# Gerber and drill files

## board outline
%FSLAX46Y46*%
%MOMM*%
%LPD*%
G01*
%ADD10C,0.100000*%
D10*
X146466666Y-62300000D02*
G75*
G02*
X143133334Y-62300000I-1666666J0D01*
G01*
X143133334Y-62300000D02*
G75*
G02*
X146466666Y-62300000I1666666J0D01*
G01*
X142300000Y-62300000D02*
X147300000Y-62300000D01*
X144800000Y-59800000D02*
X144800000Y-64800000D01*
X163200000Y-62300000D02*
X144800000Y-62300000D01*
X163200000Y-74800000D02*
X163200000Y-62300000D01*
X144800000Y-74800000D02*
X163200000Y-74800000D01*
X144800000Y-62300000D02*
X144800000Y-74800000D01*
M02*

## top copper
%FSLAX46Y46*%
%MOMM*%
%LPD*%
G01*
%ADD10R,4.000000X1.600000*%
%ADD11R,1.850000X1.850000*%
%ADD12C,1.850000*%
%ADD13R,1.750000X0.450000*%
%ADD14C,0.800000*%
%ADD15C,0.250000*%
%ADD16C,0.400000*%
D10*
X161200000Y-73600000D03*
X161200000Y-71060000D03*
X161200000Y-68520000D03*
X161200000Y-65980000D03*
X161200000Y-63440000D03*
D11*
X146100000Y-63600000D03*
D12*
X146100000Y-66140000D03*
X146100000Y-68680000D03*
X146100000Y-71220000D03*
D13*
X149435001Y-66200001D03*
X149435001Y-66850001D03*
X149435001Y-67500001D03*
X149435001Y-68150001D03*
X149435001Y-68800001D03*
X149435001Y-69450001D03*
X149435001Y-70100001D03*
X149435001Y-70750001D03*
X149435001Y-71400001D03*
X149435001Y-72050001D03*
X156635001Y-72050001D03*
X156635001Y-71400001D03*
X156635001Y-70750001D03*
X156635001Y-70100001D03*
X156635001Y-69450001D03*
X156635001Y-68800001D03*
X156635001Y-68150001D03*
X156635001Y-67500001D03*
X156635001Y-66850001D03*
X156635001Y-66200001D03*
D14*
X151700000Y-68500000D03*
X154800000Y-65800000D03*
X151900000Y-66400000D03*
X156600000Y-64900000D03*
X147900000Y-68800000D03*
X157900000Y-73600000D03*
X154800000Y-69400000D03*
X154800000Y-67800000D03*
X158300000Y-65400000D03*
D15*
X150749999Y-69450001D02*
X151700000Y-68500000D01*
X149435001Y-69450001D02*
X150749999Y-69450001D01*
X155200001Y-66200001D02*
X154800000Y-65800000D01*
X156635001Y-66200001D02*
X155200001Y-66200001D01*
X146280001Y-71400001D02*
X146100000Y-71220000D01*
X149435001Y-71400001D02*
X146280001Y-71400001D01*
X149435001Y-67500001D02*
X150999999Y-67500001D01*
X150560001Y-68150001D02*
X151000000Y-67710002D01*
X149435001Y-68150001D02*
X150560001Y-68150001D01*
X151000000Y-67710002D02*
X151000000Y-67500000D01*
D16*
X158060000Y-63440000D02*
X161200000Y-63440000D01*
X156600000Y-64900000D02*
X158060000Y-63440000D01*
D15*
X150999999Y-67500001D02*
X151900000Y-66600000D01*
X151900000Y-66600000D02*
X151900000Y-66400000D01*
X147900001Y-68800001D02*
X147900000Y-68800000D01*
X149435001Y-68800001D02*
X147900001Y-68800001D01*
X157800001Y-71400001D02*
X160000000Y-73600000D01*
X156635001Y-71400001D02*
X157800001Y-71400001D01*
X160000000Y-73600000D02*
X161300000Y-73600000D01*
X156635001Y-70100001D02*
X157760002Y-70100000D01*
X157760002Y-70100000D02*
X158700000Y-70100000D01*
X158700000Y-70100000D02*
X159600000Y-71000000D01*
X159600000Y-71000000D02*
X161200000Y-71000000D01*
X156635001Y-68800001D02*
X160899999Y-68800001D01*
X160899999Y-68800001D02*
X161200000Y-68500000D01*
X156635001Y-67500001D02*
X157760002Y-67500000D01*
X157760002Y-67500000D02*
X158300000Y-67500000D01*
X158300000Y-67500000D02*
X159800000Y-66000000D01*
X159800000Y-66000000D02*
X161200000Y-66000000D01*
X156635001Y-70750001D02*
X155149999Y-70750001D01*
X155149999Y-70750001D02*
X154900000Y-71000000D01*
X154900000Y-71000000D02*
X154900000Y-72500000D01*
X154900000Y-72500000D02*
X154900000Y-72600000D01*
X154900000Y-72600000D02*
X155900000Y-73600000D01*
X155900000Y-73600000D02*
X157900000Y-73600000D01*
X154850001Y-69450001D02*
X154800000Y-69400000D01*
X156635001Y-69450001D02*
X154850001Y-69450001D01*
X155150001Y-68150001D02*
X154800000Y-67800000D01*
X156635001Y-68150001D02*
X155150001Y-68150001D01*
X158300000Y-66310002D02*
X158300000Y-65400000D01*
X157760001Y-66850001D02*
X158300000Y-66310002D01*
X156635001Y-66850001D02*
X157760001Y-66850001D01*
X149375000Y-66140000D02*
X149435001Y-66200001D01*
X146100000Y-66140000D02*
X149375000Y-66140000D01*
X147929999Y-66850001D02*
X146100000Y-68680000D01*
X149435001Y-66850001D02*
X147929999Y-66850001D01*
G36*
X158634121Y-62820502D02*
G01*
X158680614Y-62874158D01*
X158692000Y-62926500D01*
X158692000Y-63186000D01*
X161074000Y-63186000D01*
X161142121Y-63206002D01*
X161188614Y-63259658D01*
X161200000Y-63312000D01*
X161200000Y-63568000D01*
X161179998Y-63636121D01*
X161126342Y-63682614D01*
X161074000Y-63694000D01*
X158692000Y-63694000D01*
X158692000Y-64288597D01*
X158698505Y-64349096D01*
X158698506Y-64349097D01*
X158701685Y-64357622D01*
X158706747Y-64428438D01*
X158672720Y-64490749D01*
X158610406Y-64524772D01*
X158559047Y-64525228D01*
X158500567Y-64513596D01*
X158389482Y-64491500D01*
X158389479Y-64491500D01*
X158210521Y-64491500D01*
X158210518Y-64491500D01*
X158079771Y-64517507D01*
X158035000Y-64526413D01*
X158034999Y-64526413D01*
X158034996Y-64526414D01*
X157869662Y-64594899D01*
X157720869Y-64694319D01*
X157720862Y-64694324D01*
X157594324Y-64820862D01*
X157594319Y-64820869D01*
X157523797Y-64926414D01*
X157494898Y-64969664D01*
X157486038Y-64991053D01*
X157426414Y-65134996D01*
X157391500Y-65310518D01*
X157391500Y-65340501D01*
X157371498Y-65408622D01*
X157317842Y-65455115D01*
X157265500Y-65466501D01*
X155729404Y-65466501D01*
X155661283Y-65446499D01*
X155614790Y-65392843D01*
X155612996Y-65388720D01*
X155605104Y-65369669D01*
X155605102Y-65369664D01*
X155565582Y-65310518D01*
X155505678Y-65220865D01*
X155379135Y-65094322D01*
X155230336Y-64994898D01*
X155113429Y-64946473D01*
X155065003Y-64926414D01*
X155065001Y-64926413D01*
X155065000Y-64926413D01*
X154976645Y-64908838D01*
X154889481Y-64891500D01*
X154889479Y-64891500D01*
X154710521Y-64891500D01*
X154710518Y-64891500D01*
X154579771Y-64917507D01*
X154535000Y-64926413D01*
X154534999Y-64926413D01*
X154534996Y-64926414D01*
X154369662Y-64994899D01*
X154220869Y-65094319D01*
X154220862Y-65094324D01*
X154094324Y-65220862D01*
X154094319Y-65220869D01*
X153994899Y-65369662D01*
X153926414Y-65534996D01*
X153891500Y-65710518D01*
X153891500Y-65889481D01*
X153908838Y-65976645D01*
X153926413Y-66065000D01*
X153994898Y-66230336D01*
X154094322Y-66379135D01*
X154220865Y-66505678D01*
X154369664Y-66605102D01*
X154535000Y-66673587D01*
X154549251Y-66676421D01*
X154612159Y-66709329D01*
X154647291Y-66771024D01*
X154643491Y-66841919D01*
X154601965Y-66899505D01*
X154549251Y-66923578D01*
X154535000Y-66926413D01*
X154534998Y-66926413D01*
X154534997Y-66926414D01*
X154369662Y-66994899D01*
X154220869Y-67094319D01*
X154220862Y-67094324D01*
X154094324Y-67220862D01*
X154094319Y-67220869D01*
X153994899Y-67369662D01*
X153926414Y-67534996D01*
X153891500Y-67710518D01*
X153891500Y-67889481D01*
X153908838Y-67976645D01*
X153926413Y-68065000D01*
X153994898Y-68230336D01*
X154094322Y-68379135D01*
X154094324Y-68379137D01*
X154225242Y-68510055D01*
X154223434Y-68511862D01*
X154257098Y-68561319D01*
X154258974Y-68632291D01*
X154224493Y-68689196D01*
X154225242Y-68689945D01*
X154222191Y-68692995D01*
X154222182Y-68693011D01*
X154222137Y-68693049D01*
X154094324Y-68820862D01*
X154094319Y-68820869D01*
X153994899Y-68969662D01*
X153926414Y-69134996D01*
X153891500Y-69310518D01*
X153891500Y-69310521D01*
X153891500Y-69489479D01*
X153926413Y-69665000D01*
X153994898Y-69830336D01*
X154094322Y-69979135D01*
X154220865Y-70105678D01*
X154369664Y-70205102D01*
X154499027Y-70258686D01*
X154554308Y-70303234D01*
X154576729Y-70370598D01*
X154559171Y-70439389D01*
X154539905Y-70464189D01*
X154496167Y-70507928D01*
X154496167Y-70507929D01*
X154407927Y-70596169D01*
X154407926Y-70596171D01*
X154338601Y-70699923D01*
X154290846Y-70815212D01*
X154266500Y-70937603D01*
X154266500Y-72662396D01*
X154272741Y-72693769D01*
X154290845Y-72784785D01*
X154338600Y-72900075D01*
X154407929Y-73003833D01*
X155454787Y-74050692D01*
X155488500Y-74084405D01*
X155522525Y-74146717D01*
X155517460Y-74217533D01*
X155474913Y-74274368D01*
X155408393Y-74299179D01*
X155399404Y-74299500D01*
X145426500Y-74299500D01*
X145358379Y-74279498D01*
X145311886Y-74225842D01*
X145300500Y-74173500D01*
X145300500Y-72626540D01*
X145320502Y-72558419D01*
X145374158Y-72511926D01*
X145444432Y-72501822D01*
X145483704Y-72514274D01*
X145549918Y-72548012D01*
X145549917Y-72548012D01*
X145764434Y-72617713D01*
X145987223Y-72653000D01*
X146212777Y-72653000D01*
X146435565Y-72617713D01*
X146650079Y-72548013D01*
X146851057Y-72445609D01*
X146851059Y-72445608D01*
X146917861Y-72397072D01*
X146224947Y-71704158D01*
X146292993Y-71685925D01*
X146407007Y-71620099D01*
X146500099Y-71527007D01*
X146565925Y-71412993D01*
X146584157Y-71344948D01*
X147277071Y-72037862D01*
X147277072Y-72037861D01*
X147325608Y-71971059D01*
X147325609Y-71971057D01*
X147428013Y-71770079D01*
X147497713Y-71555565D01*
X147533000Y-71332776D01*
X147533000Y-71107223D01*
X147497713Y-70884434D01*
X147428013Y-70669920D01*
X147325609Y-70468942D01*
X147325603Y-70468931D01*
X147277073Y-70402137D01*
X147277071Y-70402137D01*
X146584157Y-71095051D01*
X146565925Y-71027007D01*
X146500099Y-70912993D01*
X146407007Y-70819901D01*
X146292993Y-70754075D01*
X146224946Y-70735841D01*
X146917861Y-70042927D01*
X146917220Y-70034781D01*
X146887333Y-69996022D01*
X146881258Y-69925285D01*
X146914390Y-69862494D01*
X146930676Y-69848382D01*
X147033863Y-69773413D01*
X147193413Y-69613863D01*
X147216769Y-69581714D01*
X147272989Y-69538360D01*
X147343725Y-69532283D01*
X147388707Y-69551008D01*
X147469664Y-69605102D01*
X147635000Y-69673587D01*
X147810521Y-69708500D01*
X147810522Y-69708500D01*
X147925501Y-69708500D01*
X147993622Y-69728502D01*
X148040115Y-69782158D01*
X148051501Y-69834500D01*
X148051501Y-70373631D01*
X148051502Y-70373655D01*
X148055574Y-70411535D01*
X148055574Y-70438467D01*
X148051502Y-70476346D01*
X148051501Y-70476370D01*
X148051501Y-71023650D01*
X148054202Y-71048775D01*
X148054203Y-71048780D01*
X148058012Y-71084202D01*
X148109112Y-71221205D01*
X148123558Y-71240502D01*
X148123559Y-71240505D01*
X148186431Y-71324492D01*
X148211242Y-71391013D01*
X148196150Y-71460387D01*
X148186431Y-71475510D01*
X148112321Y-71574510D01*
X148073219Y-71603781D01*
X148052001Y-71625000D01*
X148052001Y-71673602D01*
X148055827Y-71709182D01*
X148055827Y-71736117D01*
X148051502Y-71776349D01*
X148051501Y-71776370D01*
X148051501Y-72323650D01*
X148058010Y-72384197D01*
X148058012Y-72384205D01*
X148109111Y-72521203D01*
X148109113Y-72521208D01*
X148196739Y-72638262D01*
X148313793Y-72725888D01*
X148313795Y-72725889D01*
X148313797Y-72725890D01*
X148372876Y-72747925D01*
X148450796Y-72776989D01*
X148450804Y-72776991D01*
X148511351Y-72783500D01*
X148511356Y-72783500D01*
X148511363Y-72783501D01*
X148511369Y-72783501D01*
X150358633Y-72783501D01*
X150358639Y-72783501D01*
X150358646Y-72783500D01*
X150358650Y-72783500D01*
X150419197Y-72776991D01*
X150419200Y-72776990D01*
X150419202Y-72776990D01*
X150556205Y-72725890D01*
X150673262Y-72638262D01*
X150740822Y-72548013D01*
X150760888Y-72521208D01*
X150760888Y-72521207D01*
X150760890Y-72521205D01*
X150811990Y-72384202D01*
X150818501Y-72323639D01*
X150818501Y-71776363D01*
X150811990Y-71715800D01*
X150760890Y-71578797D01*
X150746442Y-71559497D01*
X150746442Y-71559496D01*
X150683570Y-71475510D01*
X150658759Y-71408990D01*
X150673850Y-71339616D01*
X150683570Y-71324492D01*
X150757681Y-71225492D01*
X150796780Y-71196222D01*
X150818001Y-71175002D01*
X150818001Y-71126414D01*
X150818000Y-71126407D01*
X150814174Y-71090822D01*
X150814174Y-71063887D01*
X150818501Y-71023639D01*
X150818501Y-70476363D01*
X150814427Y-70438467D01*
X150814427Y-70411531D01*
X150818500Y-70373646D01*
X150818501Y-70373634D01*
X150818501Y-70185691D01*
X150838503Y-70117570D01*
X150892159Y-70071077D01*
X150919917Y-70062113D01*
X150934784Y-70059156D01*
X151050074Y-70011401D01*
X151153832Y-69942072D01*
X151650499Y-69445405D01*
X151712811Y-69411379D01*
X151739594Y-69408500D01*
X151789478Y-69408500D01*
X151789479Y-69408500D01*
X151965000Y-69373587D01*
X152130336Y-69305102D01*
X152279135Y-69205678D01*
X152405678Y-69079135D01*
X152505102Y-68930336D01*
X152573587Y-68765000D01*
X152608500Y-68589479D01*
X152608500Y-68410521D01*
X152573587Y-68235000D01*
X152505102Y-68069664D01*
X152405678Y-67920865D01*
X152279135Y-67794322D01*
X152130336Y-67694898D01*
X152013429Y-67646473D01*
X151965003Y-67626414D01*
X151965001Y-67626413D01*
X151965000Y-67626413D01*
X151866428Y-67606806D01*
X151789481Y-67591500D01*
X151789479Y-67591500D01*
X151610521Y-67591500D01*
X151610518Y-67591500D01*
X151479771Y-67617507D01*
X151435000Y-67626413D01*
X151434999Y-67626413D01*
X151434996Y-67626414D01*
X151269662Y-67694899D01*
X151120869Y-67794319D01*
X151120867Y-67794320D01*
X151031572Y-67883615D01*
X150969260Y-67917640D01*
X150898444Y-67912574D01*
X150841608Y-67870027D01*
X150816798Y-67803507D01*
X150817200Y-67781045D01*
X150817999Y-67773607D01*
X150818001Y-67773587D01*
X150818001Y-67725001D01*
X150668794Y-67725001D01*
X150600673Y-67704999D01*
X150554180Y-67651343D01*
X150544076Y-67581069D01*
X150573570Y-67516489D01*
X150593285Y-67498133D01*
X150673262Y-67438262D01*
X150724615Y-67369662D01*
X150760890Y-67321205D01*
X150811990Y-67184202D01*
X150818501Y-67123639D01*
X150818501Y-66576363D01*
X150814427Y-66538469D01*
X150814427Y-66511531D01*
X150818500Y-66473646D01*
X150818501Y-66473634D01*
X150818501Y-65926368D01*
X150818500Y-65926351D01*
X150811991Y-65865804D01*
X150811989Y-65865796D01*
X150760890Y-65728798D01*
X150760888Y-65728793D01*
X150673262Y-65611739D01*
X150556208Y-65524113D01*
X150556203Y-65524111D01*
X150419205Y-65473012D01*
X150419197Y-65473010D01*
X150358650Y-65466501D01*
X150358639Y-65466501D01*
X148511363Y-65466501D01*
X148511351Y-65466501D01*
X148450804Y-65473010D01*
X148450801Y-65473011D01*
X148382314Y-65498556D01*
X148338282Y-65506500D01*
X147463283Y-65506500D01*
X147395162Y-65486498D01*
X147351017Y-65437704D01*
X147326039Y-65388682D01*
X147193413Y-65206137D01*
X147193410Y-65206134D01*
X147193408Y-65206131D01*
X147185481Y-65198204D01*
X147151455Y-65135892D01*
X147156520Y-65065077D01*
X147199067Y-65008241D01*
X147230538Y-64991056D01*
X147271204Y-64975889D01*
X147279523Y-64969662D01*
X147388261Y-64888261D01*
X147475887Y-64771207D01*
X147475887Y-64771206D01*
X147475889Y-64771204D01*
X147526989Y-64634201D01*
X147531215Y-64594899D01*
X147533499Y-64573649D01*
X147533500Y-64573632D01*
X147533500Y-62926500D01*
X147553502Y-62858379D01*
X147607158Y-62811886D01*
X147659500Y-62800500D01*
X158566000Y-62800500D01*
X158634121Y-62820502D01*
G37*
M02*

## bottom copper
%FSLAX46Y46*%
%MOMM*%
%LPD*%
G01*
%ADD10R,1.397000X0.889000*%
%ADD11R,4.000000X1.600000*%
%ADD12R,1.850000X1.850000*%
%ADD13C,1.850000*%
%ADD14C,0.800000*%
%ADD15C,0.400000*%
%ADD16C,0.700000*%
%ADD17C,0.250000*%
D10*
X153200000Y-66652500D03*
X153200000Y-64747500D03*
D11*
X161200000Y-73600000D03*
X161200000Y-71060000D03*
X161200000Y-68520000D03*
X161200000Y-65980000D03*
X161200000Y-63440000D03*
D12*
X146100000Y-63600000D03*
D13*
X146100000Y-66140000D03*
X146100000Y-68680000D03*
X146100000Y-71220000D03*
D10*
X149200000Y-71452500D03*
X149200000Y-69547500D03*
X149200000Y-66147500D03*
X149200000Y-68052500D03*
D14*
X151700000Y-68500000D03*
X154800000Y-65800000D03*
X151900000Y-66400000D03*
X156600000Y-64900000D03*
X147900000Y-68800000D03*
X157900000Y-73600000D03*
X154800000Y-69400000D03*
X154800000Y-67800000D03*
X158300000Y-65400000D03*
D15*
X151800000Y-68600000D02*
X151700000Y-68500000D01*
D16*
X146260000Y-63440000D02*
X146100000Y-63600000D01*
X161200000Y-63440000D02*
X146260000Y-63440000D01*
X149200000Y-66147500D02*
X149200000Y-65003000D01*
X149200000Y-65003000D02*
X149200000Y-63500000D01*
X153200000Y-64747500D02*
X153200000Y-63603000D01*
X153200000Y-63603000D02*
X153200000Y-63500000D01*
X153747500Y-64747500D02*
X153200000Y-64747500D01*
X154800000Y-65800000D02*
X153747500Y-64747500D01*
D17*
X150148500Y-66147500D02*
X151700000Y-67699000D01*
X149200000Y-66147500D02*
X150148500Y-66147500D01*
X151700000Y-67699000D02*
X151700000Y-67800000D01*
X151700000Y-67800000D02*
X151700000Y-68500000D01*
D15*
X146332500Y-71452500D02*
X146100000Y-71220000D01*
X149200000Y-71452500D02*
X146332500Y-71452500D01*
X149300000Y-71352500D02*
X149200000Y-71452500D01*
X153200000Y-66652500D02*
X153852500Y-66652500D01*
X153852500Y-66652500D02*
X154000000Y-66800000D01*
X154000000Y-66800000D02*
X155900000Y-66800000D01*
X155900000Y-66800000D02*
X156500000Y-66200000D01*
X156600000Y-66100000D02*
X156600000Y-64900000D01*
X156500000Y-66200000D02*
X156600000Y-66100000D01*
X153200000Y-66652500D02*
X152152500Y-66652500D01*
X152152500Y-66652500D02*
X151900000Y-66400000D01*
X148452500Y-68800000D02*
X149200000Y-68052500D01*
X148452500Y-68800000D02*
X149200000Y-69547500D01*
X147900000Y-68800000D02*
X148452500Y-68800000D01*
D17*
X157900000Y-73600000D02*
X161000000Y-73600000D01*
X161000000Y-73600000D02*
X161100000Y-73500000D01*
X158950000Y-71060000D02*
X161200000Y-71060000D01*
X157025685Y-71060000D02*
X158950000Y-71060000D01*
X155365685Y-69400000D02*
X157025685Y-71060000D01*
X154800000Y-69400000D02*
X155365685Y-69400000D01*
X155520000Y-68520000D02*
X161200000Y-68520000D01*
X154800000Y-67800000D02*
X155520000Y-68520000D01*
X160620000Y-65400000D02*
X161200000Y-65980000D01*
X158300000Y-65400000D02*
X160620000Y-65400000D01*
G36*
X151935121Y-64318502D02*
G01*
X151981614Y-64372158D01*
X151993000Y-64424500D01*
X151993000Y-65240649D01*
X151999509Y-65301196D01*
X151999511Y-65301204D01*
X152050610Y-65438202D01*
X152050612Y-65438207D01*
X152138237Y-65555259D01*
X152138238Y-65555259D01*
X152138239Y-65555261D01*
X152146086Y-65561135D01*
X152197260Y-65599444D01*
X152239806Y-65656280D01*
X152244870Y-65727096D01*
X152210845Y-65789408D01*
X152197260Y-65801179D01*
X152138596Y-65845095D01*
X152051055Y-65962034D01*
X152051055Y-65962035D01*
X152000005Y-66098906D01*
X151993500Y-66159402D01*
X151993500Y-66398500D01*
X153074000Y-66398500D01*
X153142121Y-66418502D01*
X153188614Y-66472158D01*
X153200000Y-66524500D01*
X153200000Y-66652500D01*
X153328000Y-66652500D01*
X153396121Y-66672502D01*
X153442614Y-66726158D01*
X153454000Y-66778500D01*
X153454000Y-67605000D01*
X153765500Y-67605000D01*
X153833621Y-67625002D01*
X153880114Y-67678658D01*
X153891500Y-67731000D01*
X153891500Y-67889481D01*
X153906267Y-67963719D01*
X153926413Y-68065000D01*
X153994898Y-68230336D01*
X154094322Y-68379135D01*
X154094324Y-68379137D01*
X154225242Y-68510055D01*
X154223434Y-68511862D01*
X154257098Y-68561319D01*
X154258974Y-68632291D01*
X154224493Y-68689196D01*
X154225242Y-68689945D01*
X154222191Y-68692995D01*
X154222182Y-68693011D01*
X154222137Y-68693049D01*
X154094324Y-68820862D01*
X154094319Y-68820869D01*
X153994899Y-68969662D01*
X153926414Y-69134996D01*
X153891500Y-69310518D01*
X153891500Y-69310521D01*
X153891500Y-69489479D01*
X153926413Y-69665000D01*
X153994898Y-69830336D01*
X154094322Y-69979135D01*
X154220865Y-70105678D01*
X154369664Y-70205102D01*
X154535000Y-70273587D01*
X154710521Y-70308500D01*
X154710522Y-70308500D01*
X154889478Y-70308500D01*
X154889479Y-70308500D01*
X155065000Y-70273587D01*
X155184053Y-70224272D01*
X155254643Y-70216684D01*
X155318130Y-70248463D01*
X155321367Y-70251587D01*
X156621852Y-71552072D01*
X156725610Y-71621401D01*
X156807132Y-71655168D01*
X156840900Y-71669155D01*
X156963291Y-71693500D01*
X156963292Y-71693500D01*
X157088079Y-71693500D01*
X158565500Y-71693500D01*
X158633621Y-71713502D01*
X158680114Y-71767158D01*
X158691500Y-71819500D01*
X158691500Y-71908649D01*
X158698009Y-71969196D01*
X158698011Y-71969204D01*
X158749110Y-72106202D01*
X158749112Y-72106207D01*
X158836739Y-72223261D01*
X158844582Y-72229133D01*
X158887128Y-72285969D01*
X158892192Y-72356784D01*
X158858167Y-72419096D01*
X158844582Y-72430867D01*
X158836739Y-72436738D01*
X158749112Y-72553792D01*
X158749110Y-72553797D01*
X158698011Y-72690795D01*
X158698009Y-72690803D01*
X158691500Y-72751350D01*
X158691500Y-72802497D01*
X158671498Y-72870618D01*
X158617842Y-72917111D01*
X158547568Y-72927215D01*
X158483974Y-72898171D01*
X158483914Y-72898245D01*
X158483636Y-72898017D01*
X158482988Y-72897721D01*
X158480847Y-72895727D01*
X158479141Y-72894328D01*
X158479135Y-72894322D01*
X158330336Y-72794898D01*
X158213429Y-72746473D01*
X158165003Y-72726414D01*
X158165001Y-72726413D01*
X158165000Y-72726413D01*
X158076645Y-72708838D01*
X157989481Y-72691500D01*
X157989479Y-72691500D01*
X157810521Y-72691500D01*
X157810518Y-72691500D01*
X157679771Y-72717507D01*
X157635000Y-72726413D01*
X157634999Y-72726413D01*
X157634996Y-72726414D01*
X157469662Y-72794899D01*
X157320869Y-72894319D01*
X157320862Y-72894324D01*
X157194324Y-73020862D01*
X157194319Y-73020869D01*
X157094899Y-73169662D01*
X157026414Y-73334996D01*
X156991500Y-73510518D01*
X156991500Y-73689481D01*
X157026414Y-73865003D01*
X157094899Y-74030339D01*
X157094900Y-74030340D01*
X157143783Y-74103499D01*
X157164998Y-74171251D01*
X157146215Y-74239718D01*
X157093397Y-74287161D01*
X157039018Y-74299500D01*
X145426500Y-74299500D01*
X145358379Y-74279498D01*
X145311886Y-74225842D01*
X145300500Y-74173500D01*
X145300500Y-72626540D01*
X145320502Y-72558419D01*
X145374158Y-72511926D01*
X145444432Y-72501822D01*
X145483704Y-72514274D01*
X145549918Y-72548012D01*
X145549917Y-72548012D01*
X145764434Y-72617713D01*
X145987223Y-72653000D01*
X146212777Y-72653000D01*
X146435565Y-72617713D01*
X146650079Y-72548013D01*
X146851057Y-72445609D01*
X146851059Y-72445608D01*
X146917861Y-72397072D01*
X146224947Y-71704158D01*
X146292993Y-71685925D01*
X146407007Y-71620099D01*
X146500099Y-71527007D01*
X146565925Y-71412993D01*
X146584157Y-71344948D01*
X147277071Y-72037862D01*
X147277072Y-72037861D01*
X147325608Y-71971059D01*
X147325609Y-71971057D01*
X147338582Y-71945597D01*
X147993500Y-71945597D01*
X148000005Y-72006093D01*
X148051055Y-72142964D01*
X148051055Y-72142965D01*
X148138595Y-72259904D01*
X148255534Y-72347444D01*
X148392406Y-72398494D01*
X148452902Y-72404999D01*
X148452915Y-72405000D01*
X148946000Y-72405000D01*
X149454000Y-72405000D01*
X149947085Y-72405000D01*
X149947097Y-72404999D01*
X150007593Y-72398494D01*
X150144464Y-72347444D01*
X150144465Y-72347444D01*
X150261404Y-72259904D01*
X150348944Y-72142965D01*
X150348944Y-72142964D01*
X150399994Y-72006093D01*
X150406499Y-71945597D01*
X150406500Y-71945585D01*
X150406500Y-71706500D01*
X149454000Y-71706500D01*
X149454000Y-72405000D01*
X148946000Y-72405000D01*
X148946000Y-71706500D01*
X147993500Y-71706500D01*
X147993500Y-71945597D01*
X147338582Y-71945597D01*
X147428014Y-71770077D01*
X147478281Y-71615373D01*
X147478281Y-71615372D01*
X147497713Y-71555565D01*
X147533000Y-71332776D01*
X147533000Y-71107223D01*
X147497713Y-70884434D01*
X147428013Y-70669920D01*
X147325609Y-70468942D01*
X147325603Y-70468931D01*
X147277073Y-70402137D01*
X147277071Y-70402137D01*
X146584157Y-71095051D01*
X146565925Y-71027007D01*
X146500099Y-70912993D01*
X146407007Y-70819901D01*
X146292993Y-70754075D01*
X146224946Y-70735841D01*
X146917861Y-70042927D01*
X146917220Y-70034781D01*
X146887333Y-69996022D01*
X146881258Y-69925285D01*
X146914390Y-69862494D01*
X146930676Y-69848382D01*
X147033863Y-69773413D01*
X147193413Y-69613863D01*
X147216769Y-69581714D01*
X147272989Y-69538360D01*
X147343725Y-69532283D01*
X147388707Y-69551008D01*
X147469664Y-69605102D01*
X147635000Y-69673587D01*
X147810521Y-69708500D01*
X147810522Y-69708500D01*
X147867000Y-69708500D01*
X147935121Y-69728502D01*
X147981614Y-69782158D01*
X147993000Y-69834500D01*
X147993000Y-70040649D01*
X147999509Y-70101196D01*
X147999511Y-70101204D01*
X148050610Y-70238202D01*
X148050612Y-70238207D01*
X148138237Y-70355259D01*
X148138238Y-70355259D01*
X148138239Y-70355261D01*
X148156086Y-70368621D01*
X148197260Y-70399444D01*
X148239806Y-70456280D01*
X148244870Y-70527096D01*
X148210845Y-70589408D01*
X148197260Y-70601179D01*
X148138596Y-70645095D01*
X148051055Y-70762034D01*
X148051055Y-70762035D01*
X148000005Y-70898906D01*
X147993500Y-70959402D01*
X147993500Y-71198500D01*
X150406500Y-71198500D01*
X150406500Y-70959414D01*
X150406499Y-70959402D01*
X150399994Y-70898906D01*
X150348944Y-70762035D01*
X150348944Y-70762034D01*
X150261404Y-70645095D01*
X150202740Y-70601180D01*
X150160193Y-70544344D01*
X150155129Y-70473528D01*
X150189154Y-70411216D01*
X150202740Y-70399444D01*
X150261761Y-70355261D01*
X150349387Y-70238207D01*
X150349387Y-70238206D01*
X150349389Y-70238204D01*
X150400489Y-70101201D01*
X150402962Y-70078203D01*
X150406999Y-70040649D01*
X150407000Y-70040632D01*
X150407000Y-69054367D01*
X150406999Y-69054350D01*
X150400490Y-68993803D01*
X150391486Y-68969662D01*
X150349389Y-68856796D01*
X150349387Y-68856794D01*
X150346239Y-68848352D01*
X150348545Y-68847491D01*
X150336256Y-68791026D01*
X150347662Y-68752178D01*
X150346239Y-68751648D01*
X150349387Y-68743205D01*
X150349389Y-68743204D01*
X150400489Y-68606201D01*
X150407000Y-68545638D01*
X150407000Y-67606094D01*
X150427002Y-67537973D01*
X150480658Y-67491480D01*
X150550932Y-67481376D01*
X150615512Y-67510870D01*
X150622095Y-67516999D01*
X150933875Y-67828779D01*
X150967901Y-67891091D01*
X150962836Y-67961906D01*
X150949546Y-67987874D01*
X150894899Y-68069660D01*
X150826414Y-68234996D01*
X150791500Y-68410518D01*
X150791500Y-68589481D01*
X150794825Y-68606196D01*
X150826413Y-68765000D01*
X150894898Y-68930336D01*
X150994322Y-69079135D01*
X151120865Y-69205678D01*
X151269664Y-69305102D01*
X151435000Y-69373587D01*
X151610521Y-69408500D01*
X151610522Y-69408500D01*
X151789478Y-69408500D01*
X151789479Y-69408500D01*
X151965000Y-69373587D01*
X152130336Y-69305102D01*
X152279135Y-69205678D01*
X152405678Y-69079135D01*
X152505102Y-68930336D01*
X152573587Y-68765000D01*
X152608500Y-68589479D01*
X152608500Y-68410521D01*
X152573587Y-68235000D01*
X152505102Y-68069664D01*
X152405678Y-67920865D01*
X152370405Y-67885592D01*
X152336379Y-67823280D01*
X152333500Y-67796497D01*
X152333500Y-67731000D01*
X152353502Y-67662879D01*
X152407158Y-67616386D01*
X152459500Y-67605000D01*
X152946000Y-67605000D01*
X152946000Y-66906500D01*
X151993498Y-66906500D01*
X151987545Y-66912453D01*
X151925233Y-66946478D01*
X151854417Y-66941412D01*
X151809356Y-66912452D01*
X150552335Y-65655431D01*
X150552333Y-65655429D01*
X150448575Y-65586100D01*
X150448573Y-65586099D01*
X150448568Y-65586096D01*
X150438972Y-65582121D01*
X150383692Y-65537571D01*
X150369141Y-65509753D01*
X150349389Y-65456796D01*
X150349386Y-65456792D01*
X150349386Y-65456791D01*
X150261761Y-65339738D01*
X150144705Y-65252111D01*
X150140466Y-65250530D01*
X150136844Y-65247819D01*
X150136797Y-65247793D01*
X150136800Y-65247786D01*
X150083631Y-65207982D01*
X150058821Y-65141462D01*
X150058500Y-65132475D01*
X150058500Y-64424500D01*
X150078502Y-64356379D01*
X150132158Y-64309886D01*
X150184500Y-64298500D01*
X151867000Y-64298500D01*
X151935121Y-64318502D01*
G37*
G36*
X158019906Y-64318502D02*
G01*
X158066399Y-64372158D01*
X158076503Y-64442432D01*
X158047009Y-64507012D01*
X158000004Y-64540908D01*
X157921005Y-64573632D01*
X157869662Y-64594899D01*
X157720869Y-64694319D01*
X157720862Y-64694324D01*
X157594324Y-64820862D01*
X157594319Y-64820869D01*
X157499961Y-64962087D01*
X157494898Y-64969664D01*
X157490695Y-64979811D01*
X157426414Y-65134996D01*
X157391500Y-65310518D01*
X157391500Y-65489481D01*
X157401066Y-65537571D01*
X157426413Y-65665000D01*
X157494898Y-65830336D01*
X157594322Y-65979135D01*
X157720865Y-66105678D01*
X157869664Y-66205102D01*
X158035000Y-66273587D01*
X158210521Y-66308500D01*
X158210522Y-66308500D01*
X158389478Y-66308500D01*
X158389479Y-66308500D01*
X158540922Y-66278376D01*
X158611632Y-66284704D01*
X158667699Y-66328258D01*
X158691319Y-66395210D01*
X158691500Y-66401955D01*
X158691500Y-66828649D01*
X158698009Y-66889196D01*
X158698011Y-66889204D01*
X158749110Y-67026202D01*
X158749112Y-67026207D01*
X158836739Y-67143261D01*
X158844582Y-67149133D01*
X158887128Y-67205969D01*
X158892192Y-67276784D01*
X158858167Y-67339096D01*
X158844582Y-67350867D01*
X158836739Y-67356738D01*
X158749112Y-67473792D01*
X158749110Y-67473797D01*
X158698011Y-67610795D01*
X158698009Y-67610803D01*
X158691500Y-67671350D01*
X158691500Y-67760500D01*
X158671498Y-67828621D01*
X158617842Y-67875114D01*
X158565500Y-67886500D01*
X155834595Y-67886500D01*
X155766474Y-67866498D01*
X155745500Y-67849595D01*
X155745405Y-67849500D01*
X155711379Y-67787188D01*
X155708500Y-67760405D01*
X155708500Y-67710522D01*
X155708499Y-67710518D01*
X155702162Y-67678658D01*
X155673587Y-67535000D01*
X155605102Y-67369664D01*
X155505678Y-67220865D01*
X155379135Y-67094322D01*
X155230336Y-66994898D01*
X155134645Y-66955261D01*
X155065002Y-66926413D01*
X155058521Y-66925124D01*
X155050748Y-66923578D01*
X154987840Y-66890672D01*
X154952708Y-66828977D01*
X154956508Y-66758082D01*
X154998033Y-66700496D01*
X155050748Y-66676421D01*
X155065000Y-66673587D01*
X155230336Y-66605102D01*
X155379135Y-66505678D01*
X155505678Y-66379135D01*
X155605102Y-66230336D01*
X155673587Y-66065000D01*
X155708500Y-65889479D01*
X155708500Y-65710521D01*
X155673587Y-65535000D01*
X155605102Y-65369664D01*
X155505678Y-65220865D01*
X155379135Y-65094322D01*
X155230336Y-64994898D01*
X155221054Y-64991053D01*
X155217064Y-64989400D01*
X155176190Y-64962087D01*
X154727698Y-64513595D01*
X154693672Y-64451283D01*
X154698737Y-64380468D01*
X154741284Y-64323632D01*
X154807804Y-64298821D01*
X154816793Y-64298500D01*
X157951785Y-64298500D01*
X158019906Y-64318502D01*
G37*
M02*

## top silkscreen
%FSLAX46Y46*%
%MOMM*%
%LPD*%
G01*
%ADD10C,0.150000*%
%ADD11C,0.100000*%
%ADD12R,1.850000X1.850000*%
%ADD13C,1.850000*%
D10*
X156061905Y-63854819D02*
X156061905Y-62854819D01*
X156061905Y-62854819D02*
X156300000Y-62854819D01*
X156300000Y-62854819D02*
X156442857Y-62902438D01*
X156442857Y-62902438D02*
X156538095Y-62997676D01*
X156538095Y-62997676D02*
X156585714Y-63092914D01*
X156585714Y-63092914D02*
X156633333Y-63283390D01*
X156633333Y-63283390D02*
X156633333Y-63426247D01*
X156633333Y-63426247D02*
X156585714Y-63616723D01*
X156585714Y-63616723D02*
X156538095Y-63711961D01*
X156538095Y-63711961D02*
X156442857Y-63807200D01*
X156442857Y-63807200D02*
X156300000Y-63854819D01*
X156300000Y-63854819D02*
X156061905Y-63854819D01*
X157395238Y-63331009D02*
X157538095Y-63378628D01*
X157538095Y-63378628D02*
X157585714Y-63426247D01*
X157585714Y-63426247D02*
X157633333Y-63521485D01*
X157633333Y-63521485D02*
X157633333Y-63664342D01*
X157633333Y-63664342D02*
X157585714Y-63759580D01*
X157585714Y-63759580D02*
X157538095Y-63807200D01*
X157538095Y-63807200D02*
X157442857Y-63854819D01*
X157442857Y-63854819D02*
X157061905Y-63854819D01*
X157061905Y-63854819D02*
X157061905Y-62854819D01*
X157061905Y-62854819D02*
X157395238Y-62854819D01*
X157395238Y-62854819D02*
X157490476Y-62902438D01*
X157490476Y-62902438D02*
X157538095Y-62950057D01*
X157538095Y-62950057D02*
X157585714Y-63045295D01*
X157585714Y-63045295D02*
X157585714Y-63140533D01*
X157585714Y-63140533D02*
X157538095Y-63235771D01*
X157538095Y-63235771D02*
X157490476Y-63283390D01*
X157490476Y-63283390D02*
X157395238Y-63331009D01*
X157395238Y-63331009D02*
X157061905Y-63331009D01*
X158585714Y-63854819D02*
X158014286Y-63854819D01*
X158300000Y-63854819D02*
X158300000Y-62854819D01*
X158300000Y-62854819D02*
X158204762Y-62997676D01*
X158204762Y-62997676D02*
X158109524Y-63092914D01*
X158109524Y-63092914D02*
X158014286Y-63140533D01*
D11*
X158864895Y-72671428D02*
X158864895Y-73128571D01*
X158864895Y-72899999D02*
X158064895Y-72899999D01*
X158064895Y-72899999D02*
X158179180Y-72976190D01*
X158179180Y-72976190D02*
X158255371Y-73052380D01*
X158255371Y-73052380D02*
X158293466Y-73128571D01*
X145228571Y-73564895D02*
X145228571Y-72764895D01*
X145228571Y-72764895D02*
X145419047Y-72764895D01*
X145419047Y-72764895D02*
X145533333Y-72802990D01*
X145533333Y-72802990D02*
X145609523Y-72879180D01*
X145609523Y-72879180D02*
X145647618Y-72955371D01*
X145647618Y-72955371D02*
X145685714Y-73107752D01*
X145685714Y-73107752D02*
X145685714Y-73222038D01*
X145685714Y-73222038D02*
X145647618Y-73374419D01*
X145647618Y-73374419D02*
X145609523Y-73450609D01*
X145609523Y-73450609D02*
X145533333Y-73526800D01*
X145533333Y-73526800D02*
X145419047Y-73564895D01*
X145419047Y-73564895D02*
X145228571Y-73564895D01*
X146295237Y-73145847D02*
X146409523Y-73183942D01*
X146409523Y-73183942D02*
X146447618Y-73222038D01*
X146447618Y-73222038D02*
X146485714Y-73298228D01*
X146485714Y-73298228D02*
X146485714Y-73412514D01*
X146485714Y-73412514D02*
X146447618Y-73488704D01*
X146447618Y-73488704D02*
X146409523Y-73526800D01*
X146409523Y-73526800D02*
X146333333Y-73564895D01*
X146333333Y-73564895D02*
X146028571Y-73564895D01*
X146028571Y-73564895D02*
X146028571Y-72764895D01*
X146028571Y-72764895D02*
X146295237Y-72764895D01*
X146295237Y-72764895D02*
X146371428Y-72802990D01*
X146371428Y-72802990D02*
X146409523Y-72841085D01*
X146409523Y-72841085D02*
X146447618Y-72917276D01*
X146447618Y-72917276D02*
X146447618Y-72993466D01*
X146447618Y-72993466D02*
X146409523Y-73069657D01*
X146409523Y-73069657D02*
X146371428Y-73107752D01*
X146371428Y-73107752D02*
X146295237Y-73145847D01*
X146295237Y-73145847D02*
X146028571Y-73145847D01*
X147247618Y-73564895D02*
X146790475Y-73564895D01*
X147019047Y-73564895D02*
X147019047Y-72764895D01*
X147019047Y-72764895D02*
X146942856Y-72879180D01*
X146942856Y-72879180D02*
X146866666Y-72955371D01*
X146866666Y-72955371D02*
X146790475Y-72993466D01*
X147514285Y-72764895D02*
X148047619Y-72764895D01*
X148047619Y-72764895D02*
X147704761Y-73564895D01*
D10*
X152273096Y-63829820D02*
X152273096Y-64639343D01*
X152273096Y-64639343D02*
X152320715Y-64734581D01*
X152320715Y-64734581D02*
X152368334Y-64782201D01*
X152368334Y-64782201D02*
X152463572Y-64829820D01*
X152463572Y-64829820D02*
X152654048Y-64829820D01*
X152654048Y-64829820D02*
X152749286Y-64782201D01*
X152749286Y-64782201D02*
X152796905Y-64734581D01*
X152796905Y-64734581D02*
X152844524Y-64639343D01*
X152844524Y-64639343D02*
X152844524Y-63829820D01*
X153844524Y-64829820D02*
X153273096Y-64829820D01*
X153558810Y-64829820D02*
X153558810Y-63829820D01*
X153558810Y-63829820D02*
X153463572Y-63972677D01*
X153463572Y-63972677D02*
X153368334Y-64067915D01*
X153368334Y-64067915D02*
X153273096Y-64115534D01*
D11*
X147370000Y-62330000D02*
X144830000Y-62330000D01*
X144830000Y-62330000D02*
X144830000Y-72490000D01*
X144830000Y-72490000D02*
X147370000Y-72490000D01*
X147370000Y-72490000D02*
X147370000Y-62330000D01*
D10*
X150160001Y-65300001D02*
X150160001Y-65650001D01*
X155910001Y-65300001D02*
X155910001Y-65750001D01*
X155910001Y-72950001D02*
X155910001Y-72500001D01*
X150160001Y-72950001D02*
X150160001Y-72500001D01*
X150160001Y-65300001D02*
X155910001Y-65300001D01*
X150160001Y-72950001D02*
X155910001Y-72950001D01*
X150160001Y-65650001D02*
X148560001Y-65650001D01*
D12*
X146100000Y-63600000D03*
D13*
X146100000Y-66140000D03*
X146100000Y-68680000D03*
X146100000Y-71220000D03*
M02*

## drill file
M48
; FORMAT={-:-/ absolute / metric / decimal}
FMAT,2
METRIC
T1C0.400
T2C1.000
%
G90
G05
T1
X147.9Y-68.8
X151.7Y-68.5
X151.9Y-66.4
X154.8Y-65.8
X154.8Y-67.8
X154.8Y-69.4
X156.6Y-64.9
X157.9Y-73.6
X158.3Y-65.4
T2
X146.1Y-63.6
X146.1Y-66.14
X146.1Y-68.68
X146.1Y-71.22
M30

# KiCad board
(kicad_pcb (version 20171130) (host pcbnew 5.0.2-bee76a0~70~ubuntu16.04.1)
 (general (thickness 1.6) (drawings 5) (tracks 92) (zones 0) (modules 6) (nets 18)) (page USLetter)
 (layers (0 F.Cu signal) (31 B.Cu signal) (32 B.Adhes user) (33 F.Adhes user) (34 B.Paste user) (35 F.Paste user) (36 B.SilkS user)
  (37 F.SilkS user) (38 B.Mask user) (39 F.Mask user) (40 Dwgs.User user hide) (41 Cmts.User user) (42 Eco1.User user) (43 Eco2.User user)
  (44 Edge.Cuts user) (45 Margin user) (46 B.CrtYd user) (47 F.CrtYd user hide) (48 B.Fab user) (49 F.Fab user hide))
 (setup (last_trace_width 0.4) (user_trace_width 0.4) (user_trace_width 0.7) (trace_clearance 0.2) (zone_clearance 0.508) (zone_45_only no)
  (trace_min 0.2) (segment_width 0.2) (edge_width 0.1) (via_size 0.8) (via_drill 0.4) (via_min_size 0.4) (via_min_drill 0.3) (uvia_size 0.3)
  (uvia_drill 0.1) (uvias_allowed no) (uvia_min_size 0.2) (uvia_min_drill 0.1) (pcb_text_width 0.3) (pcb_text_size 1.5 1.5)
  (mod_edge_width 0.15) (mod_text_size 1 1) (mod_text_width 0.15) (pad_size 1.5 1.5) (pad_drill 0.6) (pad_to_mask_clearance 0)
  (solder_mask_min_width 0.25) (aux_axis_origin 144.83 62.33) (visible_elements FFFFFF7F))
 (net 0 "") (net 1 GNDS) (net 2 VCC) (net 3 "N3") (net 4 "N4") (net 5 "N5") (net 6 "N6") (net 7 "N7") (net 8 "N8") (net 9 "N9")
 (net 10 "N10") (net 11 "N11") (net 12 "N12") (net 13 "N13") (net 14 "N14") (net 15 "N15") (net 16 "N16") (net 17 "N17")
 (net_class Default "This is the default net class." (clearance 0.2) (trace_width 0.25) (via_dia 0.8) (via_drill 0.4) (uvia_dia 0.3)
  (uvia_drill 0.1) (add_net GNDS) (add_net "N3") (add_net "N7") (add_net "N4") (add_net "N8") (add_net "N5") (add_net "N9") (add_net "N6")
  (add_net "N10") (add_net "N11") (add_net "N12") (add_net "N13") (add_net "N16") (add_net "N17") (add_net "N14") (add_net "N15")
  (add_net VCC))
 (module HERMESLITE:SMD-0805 (layer B.Cu) (at 153.2 65.7 90)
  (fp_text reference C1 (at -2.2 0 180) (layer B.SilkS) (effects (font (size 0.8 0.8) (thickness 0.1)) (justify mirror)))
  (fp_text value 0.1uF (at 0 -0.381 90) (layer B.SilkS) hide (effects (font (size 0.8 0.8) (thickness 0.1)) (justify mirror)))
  (pad 1 smd rect (at -0.9525 0 90) (size 0.889 1.397) (layers B.Cu B.Paste B.Mask) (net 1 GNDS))
  (pad 2 smd rect (at 0.9525 0 90) (size 0.889 1.397) (layers B.Cu B.Paste B.Mask) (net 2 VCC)))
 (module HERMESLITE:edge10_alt (layer F.Cu) (at 161.2 73.6 270)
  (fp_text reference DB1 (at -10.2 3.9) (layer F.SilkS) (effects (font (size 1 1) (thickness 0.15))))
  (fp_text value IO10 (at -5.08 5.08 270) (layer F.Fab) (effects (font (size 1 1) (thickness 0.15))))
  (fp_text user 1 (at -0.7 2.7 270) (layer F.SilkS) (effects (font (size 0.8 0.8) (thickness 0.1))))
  (pad 1 smd rect (at 0 0 270) (size 1.6 4) (layers F.Cu F.Paste F.Mask) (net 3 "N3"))
  (pad 3 smd rect (at -2.54 0 270) (size 1.6 4) (layers F.Cu F.Paste F.Mask) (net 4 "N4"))
  (pad 5 smd rect (at -5.08 0 270) (size 1.6 4) (layers F.Cu F.Paste F.Mask) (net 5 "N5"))
  (pad 7 smd rect (at -7.62 0 270) (size 1.6 4) (layers F.Cu F.Paste F.Mask) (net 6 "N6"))
  (pad 9 smd rect (at -10.16 0 270) (size 1.6 4) (layers F.Cu F.Paste F.Mask) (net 1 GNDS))
  (pad 2 smd rect (at 0 0 270) (size 1.6 4) (layers B.Cu B.Paste B.Mask) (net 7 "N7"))
  (pad 4 smd rect (at -2.54 0 270) (size 1.6 4) (layers B.Cu B.Paste B.Mask) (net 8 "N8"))
  (pad 6 smd rect (at -5.08 0 270) (size 1.6 4) (layers B.Cu B.Paste B.Mask) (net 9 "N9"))
  (pad 8 smd rect (at -7.62 0 270) (size 1.6 4) (layers B.Cu B.Paste B.Mask) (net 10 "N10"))
  (pad 10 smd rect (at -10.16 0 270) (size 1.6 4) (layers B.Cu B.Paste B.Mask) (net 2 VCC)))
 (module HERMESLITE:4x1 (layer F.Cu) (at 146.1 63.6 270)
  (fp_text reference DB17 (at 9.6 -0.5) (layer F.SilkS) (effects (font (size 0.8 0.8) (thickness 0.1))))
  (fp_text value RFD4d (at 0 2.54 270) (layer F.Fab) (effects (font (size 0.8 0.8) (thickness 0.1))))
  (fp_line (start -1.27 -1.27) (end -1.27 1.27) (layer F.SilkS) (width 0.1))
  (fp_line (start -1.27 1.27) (end 8.89 1.27) (layer F.SilkS) (width 0.1))
  (fp_line (start 8.89 1.27) (end 8.89 -1.27) (layer F.SilkS) (width 0.1))
  (fp_line (start 8.89 -1.27) (end -1.27 -1.27) (layer F.SilkS) (width 0.1))
  (pad 1 thru_hole rect (at 0 0 270) (size 1.85 1.85) (drill 1) (layers *.Cu *.Mask F.SilkS) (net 2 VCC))
  (pad 2 thru_hole circle (at 2.54 0 270) (size 1.85 1.85) (drill 1) (layers *.Cu *.Mask F.SilkS) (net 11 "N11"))
  (pad 3 thru_hole circle (at 5.08 0 270) (size 1.85 1.85) (drill 1) (layers *.Cu *.Mask F.SilkS) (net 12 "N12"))
  (pad 4 thru_hole circle (at 7.62 0 270) (size 1.85 1.85) (drill 1) (layers *.Cu *.Mask F.SilkS) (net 1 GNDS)))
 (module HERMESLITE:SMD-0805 (layer B.Cu) (at 149.2 70.5 270)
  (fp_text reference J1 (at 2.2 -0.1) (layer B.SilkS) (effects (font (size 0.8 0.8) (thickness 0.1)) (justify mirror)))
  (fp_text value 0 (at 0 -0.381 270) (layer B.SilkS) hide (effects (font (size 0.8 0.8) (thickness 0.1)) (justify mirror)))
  (pad 2 smd rect (at 0.9525 0 270) (size 0.889 1.397) (layers B.Cu B.Paste B.Mask) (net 1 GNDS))
  (pad 1 smd rect (at -0.9525 0 270) (size 0.889 1.397) (layers B.Cu B.Paste B.Mask) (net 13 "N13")))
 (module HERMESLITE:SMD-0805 (layer B.Cu) (at 149.2 67.1 270)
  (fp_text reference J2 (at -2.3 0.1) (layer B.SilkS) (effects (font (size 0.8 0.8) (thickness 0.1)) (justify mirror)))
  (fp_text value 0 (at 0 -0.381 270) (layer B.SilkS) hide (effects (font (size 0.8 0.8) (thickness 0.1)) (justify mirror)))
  (pad 1 smd rect (at -0.9525 0 270) (size 0.889 1.397) (layers B.Cu B.Paste B.Mask) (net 2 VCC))
  (pad 2 smd rect (at 0.9525 0 270) (size 0.889 1.397) (layers B.Cu B.Paste B.Mask) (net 13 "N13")))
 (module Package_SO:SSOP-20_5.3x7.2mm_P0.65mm (layer F.Cu) (at 153.035001 69.125001)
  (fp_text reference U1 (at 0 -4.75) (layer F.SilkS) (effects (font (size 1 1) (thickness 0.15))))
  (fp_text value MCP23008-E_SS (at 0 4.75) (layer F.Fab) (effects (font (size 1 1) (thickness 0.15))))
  (fp_line (start -2.875 -3.825) (end -2.875 -3.475) (layer F.SilkS) (width 0.15))
  (fp_line (start 2.875 -3.825) (end 2.875 -3.375) (layer F.SilkS) (width 0.15))
  (fp_line (start 2.875 3.825) (end 2.875 3.375) (layer F.SilkS) (width 0.15))
  (fp_line (start -2.875 3.825) (end -2.875 3.375) (layer F.SilkS) (width 0.15))
  (fp_line (start -2.875 -3.825) (end 2.875 -3.825) (layer F.SilkS) (width 0.15))
  (fp_line (start -2.875 3.825) (end 2.875 3.825) (layer F.SilkS) (width 0.15))
  (fp_line (start -2.875 -3.475) (end -4.475 -3.475) (layer F.SilkS) (width 0.15))
  (pad 1 smd rect (at -3.6 -2.925) (size 1.75 0.45) (layers F.Cu F.Paste F.Mask) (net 11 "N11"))
  (pad 2 smd rect (at -3.6 -2.275) (size 1.75 0.45) (layers F.Cu F.Paste F.Mask) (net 12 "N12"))
  (pad 3 smd rect (at -3.6 -1.625) (size 1.75 0.45) (layers F.Cu F.Paste F.Mask) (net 1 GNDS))
  (pad 4 smd rect (at -3.6 -0.975) (size 1.75 0.45) (layers F.Cu F.Paste F.Mask) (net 1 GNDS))
  (pad 5 smd rect (at -3.6 -0.325) (size 1.75 0.45) (layers F.Cu F.Paste F.Mask) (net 13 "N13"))
  (pad 6 smd rect (at -3.6 0.325) (size 1.75 0.45) (layers F.Cu F.Paste F.Mask) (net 2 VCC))
  (pad 7 smd rect (at -3.6 0.975) (size 1.75 0.45) (layers F.Cu F.Paste F.Mask) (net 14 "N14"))
  (pad 8 smd rect (at -3.6 1.625) (size 1.75 0.45) (layers F.Cu F.Paste F.Mask) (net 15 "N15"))
  (pad 9 smd rect (at -3.6 2.275) (size 1.75 0.45) (layers F.Cu F.Paste F.Mask) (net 1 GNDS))
  (pad 10 smd rect (at -3.6 2.925) (size 1.75 0.45) (layers F.Cu F.Paste F.Mask) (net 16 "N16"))
  (pad 11 smd rect (at 3.6 2.925) (size 1.75 0.45) (layers F.Cu F.Paste F.Mask) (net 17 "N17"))
  (pad 12 smd rect (at 3.6 2.275) (size 1.75 0.45) (layers F.Cu F.Paste F.Mask) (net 3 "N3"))
  (pad 13 smd rect (at 3.6 1.625) (size 1.75 0.45) (layers F.Cu F.Paste F.Mask) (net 7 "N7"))
  (pad 14 smd rect (at 3.6 0.975) (size 1.75 0.45) (layers F.Cu F.Paste F.Mask) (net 4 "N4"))
  (pad 15 smd rect (at 3.6 0.325) (size 1.75 0.45) (layers F.Cu F.Paste F.Mask) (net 8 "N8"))
  (pad 16 smd rect (at 3.6 -0.325) (size 1.75 0.45) (layers F.Cu F.Paste F.Mask) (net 5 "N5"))
  (pad 17 smd rect (at 3.6 -0.975) (size 1.75 0.45) (layers F.Cu F.Paste F.Mask) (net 9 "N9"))
  (pad 18 smd rect (at 3.6 -1.625) (size 1.75 0.45) (layers F.Cu F.Paste F.Mask) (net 6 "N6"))
  (pad 19 smd rect (at 3.6 -2.275) (size 1.75 0.45) (layers F.Cu F.Paste F.Mask) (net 10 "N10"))
  (pad 20 smd rect (at 3.6 -2.925) (size 1.75 0.45) (layers F.Cu F.Paste F.Mask) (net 2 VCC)))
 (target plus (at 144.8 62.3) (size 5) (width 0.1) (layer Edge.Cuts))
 (gr_line (start 163.2 62.3) (end 144.8 62.3) (layer Edge.Cuts) (width 0.1))
 (gr_line (start 163.2 74.8) (end 163.2 62.3) (layer Edge.Cuts) (width 0.1))
 (gr_line (start 144.8 74.8) (end 163.2 74.8) (layer Edge.Cuts) (width 0.1))
 (gr_line (start 144.8 62.3) (end 144.8 74.8) (layer Edge.Cuts) (width 0.1))
 (via (at 151.7 68.5) (size 0.8) (drill 0.4) (layers F.Cu B.Cu) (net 2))
 (segment (start 150.749999 69.450001) (end 151.7 68.5) (width 0.25) (layer F.Cu) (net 2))
 (segment (start 149.435001 69.450001) (end 150.749999 69.450001) (width 0.25) (layer F.Cu) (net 2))
 (segment (start 151.8 68.6) (end 151.7 68.5) (width 0.4) (layer B.Cu) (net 2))
 (segment (start 146.26 63.44) (end 146.1 63.6) (width 0.7) (layer B.Cu) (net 2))
 (segment (start 161.2 63.44) (end 146.26 63.44) (width 0.7) (layer B.Cu) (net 2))
 (segment (start 149.2 66.1475) (end 149.2 65.003) (width 0.7) (layer B.Cu) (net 2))
 (segment (start 149.2 65.003) (end 149.2 63.5) (width 0.7) (layer B.Cu) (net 2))
 (via (at 154.8 65.8) (size 0.8) (drill 0.4) (layers F.Cu B.Cu) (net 2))
 (segment (start 155.200001 66.200001) (end 154.8 65.8) (width 0.25) (layer F.Cu) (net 2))
 (segment (start 156.635001 66.200001) (end 155.200001 66.200001) (width 0.25) (layer F.Cu) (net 2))
 (segment (start 153.2 64.7475) (end 153.2 63.603) (width 0.7) (layer B.Cu) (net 2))
 (segment (start 153.2 63.603) (end 153.2 63.5) (width 0.7) (layer B.Cu) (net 2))
 (segment (start 153.7475 64.7475) (end 153.2 64.7475) (width 0.7) (layer B.Cu) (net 2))
 (segment (start 154.8 65.8) (end 153.7475 64.7475) (width 0.7) (layer B.Cu) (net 2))
 (segment (start 150.1485 66.1475) (end 151.7 67.699) (width 0.25) (layer B.Cu) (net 2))
 (segment (start 149.2 66.1475) (end 150.1485 66.1475) (width 0.25) (layer B.Cu) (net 2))
 (segment (start 151.7 67.699) (end 151.7 67.8) (width 0.25) (layer B.Cu) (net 2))
 (segment (start 151.7 67.8) (end 151.7 68.5) (width 0.25) (layer B.Cu) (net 2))
 (segment (start 146.280001 71.400001) (end 146.1 71.22) (width 0.25) (layer F.Cu) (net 1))
 (segment (start 149.435001 71.400001) (end 146.280001 71.400001) (width 0.25) (layer F.Cu) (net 1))
 (segment (start 146.3325 71.4525) (end 146.1 71.22) (width 0.4) (layer B.Cu) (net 1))
 (segment (start 149.2 71.4525) (end 146.3325 71.4525) (width 0.4) (layer B.Cu) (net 1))
 (segment (start 149.3 71.3525) (end 149.2 71.4525) (width 0.4) (layer B.Cu) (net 1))
 (segment (start 149.435001 67.500001) (end 150.999999 67.500001) (width 0.25) (layer F.Cu) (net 1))
 (via (at 151.9 66.4) (size 0.8) (drill 0.4) (layers F.Cu B.Cu) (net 1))
 (segment (start 150.560001 68.150001) (end 151 67.710002) (width 0.25) (layer F.Cu) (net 1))
 (segment (start 149.435001 68.150001) (end 150.560001 68.150001) (width 0.25) (layer F.Cu) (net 1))
 (segment (start 151 67.710002) (end 151 67.5) (width 0.25) (layer F.Cu) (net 1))
 (segment (start 153.2 66.6525) (end 153.8525 66.6525) (width 0.4) (layer B.Cu) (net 1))
 (segment (start 153.8525 66.6525) (end 154 66.8) (width 0.4) (layer B.Cu) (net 1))
 (segment (start 154 66.8) (end 155.9 66.8) (width 0.4) (layer B.Cu) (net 1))
 (segment (start 155.9 66.8) (end 156.5 66.2) (width 0.4) (layer B.Cu) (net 1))
 (via (at 156.6 64.9) (size 0.8) (drill 0.4) (layers F.Cu B.Cu) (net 1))
 (segment (start 156.6 66.1) (end 156.6 64.9) (width 0.4) (layer B.Cu) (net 1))
 (segment (start 156.5 66.2) (end 156.6 66.1) (width 0.4) (layer B.Cu) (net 1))
 (segment (start 158.06 63.44) (end 161.2 63.44) (width 0.4) (layer F.Cu) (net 1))
 (segment (start 156.6 64.9) (end 158.06 63.44) (width 0.4) (layer F.Cu) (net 1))
 (segment (start 150.999999 67.500001) (end 151.9 66.6) (width 0.25) (layer F.Cu) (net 1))
 (segment (start 151.9 66.6) (end 151.9 66.4) (width 0.25) (layer F.Cu) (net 1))
 (segment (start 153.2 66.6525) (end 152.1525 66.6525) (width 0.4) (layer B.Cu) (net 1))
 (segment (start 152.1525 66.6525) (end 151.9 66.4) (width 0.4) (layer B.Cu) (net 1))
 (via (at 147.9 68.8) (size 0.8) (drill 0.4) (layers F.Cu B.Cu) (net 13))
 (segment (start 147.900001 68.800001) (end 147.9 68.8) (width 0.25) (layer F.Cu) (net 13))
 (segment (start 149.435001 68.800001) (end 147.900001 68.800001) (width 0.25) (layer F.Cu) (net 13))
 (segment (start 148.4525 68.8) (end 149.2 68.0525) (width 0.4) (layer B.Cu) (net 13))
 (segment (start 148.4525 68.8) (end 149.2 69.5475) (width 0.4) (layer B.Cu) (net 13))
 (segment (start 147.9 68.8) (end 148.4525 68.8) (width 0.4) (layer B.Cu) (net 13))
 (segment (start 157.800001 71.400001) (end 160 73.6) (width 0.25) (layer F.Cu) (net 3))
 (segment (start 156.635001 71.400001) (end 157.800001 71.400001) (width 0.25) (layer F.Cu) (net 3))
 (segment (start 160 73.6) (end 161.3 73.6) (width 0.25) (layer F.Cu) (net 3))
 (segment (start 156.635001 70.100001) (end 157.760002 70.1) (width 0.25) (layer F.Cu) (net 4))
 (segment (start 157.760002 70.1) (end 158.7 70.1) (width 0.25) (layer F.Cu) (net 4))
 (segment (start 158.7 70.1) (end 159.6 71) (width 0.25) (layer F.Cu) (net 4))
 (segment (start 159.6 71) (end 161.2 71) (width 0.25) (layer F.Cu) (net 4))
 (segment (start 156.635001 68.800001) (end 160.899999 68.800001) (width 0.25) (layer F.Cu) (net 5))
 (segment (start 160.899999 68.800001) (end 161.2 68.5) (width 0.25) (layer F.Cu) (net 5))
 (segment (start 156.635001 67.500001) (end 157.760002 67.5) (width 0.25) (layer F.Cu) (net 6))
 (segment (start 157.760002 67.5) (end 158.3 67.5) (width 0.25) (layer F.Cu) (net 6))
 (segment (start 158.3 67.5) (end 159.8 66) (width 0.25) (layer F.Cu) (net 6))
 (segment (start 159.8 66) (end 161.2 66) (width 0.25) (layer F.Cu) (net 6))
 (segment (start 156.635001 70.750001) (end 155.149999 70.750001) (width 0.25) (layer F.Cu) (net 7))
 (segment (start 155.149999 70.750001) (end 154.9 71) (width 0.25) (layer F.Cu) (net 7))
 (segment (start 154.9 71) (end 154.9 72.5) (width 0.25) (layer F.Cu) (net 7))
 (segment (start 154.9 72.5) (end 154.9 72.6) (width 0.25) (layer F.Cu) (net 7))
 (segment (start 154.9 72.6) (end 155.9 73.6) (width 0.25) (layer F.Cu) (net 7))
 (via (at 157.9 73.6) (size 0.8) (drill 0.4) (layers F.Cu B.Cu) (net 7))
 (segment (start 155.9 73.6) (end 157.9 73.6) (width 0.25) (layer F.Cu) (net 7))
 (segment (start 157.9 73.6) (end 161 73.6) (width 0.25) (layer B.Cu) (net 7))
 (segment (start 161 73.6) (end 161.1 73.5) (width 0.25) (layer B.Cu) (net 7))
 (via (at 154.8 69.4) (size 0.8) (drill 0.4) (layers F.Cu B.Cu) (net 8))
 (segment (start 154.850001 69.450001) (end 154.8 69.4) (width 0.25) (layer F.Cu) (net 8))
 (segment (start 156.635001 69.450001) (end 154.850001 69.450001) (width 0.25) (layer F.Cu) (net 8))
 (segment (start 158.95 71.06) (end 161.2 71.06) (width 0.25) (layer B.Cu) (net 8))
 (segment (start 157.025685 71.06) (end 158.95 71.06) (width 0.25) (layer B.Cu) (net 8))
 (segment (start 155.365685 69.4) (end 157.025685 71.06) (width 0.25) (layer B.Cu) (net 8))
 (segment (start 154.8 69.4) (end 155.365685 69.4) (width 0.25) (layer B.Cu) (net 8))
 (segment (start 155.150001 68.150001) (end 154.8 67.8) (width 0.25) (layer F.Cu) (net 9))
 (via (at 154.8 67.8) (size 0.8) (drill 0.4) (layers F.Cu B.Cu) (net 9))
 (segment (start 156.635001 68.150001) (end 155.150001 68.150001) (width 0.25) (layer F.Cu) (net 9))
 (segment (start 155.52 68.52) (end 161.2 68.52) (width 0.25) (layer B.Cu) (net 9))
 (segment (start 154.8 67.8) (end 155.52 68.52) (width 0.25) (layer B.Cu) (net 9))
 (via (at 158.3 65.4) (size 0.8) (drill 0.4) (layers F.Cu B.Cu) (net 10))
 (segment (start 158.3 66.310002) (end 158.3 65.4) (width 0.25) (layer F.Cu) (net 10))
 (segment (start 157.760001 66.850001) (end 158.3 66.310002) (width 0.25) (layer F.Cu) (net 10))
 (segment (start 156.635001 66.850001) (end 157.760001 66.850001) (width 0.25) (layer F.Cu) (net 10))
 (segment (start 160.62 65.4) (end 161.2 65.98) (width 0.25) (layer B.Cu) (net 10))
 (segment (start 158.3 65.4) (end 160.62 65.4) (width 0.25) (layer B.Cu) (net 10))
 (segment (start 149.375 66.14) (end 149.435001 66.200001) (width 0.25) (layer F.Cu) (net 11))
 (segment (start 146.1 66.14) (end 149.375 66.14) (width 0.25) (layer F.Cu) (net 11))
 (segment (start 147.929999 66.850001) (end 146.1 68.68) (width 0.25) (layer F.Cu) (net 12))
 (segment (start 149.435001 66.850001) (end 147.929999 66.850001) (width 0.25) (layer F.Cu) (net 12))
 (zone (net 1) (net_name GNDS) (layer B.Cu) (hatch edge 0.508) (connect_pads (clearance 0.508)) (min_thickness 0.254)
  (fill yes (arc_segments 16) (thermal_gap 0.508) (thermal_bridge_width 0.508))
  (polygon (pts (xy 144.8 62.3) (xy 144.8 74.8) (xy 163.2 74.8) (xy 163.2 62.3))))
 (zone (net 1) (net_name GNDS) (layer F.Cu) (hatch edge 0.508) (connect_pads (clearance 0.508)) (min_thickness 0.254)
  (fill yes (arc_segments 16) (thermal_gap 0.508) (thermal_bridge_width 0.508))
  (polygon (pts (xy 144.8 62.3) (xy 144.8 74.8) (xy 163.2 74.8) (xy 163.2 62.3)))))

